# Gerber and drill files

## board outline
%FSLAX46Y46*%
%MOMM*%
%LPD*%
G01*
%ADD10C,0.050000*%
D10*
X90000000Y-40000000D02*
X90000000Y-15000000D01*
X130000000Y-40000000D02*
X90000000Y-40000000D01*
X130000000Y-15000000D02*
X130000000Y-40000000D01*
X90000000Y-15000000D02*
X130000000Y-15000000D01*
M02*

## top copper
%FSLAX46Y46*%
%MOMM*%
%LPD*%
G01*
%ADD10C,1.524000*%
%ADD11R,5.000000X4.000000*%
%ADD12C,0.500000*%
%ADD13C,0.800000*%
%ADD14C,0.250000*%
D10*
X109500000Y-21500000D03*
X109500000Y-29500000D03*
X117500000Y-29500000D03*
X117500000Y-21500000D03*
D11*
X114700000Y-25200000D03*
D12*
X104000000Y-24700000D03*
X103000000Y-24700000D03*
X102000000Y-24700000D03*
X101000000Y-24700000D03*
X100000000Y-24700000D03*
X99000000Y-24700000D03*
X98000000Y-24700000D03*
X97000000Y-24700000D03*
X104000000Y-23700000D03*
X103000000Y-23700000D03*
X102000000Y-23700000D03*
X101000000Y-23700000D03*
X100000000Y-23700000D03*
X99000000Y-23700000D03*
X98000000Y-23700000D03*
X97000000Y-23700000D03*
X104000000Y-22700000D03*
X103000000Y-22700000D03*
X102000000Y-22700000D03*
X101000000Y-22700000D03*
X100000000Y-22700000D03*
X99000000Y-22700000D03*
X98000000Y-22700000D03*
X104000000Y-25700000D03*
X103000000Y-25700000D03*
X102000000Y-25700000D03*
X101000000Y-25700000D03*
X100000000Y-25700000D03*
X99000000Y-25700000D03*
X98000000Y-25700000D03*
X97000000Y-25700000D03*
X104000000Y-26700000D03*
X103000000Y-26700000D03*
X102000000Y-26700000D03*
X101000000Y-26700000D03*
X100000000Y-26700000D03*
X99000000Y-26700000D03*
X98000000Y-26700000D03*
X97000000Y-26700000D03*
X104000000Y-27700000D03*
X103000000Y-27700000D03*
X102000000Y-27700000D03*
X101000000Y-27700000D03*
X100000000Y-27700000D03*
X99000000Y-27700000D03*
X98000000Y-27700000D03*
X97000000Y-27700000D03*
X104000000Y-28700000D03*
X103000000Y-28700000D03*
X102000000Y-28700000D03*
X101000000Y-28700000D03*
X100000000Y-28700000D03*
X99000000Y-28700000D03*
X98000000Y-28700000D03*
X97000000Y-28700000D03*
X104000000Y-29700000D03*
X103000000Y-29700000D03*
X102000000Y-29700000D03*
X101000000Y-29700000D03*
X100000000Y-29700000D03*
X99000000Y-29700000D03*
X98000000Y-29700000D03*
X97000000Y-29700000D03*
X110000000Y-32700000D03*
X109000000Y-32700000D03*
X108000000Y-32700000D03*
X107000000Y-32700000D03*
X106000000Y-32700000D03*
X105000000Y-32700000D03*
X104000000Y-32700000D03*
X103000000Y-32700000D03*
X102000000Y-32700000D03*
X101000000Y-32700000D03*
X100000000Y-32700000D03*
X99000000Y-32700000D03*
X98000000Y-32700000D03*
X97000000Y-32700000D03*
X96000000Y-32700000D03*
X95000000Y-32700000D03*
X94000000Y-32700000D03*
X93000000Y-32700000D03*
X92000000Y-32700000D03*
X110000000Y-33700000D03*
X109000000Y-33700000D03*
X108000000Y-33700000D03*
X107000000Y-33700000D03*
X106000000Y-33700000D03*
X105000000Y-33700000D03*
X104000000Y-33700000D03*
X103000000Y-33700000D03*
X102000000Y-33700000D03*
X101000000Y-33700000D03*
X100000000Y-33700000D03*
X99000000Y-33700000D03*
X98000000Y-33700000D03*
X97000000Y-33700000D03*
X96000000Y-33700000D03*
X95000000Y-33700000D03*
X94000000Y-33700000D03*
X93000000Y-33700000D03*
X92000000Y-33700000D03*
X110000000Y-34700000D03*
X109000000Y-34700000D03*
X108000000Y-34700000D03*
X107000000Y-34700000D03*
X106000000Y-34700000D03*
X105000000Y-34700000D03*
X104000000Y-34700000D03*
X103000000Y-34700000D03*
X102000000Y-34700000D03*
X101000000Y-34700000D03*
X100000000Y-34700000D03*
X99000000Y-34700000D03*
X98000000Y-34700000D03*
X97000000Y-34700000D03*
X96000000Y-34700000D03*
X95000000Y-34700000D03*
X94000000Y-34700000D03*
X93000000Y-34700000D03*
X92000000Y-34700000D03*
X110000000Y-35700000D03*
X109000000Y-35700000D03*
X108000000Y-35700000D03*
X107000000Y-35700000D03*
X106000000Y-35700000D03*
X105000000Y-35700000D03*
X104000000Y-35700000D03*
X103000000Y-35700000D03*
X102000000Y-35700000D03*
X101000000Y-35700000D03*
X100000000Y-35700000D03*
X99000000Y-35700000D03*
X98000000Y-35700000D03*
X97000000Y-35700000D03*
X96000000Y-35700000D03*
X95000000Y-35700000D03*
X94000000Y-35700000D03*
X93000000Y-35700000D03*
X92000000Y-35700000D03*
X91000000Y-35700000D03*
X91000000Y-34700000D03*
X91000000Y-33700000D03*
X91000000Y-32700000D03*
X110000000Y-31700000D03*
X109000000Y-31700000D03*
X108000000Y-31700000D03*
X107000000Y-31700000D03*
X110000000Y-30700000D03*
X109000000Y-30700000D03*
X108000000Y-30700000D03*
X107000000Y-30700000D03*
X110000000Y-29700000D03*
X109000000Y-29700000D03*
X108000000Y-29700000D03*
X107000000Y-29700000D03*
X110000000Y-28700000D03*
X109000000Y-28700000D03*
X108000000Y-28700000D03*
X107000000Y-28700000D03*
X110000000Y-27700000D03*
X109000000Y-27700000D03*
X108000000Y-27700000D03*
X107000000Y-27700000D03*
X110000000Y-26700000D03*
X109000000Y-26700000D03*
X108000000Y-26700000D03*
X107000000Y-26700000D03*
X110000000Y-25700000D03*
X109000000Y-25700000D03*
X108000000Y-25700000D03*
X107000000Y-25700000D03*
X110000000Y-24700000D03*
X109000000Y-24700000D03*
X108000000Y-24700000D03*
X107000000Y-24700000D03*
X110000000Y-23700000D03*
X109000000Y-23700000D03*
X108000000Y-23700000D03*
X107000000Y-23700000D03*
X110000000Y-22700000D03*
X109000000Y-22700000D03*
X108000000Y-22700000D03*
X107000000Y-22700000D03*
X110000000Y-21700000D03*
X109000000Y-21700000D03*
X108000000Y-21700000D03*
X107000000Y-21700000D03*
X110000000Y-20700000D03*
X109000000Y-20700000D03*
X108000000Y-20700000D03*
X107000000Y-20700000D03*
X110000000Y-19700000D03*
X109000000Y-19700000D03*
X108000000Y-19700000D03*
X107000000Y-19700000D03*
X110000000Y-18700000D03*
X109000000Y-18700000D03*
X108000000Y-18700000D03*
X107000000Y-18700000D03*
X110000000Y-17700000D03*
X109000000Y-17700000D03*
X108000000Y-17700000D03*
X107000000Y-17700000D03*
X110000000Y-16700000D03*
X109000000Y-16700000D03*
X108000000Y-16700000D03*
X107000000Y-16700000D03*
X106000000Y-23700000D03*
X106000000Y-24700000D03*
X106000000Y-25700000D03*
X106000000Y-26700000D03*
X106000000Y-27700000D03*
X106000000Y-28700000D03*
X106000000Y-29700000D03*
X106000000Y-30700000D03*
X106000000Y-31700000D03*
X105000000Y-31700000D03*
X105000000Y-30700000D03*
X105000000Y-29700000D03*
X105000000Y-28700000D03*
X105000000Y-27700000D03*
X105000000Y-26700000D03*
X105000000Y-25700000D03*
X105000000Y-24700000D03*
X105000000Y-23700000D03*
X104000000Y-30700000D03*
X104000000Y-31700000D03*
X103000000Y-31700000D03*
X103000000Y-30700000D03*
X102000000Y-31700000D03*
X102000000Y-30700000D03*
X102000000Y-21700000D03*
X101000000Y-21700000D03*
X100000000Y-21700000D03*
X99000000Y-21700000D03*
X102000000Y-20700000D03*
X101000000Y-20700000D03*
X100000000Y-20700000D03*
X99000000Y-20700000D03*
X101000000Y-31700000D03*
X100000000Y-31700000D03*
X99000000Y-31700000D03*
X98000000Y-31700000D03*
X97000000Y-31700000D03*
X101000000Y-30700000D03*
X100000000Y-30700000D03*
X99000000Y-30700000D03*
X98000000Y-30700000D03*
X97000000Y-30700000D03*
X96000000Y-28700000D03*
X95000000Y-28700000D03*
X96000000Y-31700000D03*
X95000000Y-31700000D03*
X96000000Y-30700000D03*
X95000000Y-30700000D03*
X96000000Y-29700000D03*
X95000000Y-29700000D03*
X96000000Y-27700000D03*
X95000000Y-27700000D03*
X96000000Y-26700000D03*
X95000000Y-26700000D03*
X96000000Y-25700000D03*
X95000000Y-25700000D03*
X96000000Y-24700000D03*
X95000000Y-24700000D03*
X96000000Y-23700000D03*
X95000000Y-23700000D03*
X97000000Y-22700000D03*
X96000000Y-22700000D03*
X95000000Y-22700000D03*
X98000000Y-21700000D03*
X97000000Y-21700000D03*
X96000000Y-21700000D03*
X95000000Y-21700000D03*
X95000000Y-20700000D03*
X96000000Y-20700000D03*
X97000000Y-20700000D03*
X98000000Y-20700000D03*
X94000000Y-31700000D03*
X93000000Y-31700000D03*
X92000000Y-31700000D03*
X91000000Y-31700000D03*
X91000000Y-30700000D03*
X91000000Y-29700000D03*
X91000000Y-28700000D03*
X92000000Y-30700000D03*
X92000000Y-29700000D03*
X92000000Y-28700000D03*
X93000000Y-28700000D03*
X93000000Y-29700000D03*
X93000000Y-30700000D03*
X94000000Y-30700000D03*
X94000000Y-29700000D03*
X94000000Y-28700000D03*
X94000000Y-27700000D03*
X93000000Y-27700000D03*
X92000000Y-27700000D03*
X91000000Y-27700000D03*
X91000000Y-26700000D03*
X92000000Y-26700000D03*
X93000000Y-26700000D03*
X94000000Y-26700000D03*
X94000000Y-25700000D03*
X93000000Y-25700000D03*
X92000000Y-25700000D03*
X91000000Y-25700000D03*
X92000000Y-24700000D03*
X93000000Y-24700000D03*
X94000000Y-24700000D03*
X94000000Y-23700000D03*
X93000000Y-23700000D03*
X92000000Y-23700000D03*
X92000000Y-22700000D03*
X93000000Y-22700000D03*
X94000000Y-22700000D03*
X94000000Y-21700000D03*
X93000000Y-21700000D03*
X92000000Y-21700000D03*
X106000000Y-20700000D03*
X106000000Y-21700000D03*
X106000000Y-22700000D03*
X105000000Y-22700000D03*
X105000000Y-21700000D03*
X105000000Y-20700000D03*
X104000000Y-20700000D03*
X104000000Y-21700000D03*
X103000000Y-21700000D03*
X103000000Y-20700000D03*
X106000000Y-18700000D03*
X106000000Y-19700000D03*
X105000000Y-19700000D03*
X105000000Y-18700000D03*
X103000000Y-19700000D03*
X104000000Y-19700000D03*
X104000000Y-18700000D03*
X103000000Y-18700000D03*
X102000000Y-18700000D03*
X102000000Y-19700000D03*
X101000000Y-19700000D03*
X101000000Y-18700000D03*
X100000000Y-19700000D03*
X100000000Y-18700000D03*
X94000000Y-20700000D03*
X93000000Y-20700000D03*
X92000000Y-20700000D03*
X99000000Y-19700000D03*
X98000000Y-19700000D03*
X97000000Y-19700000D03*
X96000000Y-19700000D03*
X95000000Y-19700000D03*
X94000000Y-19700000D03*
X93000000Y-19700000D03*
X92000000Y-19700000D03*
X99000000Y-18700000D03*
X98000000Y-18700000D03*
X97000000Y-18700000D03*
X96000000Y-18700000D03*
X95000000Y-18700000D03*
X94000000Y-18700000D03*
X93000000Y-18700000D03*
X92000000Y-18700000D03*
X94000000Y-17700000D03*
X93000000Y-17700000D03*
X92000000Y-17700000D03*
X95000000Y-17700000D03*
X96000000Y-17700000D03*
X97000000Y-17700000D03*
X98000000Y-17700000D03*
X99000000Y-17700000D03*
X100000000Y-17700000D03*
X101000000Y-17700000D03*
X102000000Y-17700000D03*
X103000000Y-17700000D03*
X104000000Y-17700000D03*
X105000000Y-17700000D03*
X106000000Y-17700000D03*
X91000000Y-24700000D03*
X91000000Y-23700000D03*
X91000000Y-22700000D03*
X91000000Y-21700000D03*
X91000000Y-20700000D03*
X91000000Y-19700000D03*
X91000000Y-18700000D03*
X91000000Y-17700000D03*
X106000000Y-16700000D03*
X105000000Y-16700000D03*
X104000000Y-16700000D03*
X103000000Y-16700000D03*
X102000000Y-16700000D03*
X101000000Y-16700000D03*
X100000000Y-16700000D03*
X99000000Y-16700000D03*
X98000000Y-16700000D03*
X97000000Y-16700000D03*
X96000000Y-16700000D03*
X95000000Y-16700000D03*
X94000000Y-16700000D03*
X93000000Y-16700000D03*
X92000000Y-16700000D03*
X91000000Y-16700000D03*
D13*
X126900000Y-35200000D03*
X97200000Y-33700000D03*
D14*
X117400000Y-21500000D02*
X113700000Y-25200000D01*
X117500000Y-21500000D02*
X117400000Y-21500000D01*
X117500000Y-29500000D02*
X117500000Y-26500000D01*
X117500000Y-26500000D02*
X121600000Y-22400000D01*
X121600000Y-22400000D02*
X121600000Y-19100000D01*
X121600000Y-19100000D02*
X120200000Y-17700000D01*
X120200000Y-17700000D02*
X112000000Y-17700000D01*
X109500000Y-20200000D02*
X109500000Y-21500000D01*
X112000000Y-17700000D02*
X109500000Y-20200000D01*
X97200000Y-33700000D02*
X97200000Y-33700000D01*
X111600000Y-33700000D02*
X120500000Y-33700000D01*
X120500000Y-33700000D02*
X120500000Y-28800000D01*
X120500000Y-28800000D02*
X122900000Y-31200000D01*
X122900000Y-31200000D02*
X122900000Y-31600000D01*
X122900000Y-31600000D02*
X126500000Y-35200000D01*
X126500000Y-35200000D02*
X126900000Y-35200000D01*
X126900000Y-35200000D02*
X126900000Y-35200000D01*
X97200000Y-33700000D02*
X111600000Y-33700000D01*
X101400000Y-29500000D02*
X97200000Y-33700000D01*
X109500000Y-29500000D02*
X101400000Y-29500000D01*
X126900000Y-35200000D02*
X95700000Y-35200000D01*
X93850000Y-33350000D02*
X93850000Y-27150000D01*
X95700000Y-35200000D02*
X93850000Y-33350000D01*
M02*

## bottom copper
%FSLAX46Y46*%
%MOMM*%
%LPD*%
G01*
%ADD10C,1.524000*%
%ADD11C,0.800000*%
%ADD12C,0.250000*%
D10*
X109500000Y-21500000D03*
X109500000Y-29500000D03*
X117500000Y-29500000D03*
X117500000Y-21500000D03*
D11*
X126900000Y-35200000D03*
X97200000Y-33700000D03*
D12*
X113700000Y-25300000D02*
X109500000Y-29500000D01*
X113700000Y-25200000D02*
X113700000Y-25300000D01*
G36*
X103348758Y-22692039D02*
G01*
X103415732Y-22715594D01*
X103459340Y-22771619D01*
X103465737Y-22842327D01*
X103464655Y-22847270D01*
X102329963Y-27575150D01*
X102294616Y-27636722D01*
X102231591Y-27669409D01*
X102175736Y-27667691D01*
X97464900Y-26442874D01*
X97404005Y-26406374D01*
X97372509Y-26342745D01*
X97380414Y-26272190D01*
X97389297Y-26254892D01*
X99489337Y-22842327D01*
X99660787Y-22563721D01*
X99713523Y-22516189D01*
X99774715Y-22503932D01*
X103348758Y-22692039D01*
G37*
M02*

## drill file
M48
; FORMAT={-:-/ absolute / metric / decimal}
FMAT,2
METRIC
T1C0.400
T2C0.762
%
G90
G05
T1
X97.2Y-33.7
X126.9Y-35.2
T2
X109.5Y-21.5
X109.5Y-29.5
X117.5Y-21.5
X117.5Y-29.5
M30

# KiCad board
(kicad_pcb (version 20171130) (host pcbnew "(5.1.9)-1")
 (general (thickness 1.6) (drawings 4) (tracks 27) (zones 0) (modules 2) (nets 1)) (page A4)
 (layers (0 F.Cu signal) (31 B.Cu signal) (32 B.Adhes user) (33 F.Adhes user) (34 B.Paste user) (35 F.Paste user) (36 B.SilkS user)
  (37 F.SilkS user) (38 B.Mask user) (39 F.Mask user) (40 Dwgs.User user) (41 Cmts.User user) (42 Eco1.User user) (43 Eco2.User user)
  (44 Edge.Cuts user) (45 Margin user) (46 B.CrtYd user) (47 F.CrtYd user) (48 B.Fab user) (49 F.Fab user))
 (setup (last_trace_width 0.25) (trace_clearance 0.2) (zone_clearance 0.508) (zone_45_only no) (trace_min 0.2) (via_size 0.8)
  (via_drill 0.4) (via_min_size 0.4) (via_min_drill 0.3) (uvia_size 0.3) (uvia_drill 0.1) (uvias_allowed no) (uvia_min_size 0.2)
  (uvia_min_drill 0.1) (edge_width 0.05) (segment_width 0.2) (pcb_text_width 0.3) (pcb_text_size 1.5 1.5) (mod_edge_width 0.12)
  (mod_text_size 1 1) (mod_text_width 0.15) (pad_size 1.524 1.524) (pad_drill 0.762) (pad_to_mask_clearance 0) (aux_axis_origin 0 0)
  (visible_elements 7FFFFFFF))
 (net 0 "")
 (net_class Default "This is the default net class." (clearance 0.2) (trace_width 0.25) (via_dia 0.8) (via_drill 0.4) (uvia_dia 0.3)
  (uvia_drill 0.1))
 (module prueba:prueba (layer F.Cu) (at 113.5 25.5)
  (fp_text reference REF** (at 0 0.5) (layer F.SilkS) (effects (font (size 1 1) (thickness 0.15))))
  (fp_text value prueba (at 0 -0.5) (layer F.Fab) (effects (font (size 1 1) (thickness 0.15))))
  (pad 5 thru_hole circle (at -4 -4 45) (size 1.524 1.524) (drill 0.762) (layers *.Cu *.Mask))
  (pad 4 thru_hole circle (at -4 4) (size 1.524 1.524) (drill 0.762) (layers *.Cu *.Mask))
  (pad 3 thru_hole circle (at 4 4) (size 1.524 1.524) (drill 0.762) (layers *.Cu *.Mask))
  (pad 2 thru_hole circle (at 4 -4) (size 1.524 1.524) (drill 0.762) (layers *.Cu *.Mask))
  (pad 1 smd rect (at 0.2 -0.3) (size 5 4) (drill (offset 1 0)) (layers F.Cu F.Paste F.Mask) (die_length 1)))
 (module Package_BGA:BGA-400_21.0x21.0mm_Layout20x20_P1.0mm (layer F.Cu) (at 100.5 26.2)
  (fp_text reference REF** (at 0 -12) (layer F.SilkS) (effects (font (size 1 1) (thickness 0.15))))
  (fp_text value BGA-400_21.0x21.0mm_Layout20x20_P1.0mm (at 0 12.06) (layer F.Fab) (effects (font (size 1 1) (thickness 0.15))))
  (pad J14 smd circle (at 3.5 -1.5) (size 0.5 0.5) (layers F.Cu F.Paste F.Mask))
  (pad J13 smd circle (at 2.5 -1.5) (size 0.5 0.5) (layers F.Cu F.Paste F.Mask))
  (pad J12 smd circle (at 1.5 -1.5) (size 0.5 0.5) (layers F.Cu F.Paste F.Mask))
  (pad J11 smd circle (at 0.5 -1.5) (size 0.5 0.5) (layers F.Cu F.Paste F.Mask))
  (pad J10 smd circle (at -0.5 -1.5) (size 0.5 0.5) (layers F.Cu F.Paste F.Mask))
  (pad J9 smd circle (at -1.5 -1.5) (size 0.5 0.5) (layers F.Cu F.Paste F.Mask))
  (pad J8 smd circle (at -2.5 -1.5) (size 0.5 0.5) (layers F.Cu F.Paste F.Mask))
  (pad J7 smd circle (at -3.5 -1.5) (size 0.5 0.5) (layers F.Cu F.Paste F.Mask))
  (pad H14 smd circle (at 3.5 -2.5) (size 0.5 0.5) (layers F.Cu F.Paste F.Mask))
  (pad H13 smd circle (at 2.5 -2.5) (size 0.5 0.5) (layers F.Cu F.Paste F.Mask))
  (pad H12 smd circle (at 1.5 -2.5) (size 0.5 0.5) (layers F.Cu F.Paste F.Mask))
  (pad H11 smd circle (at 0.5 -2.5) (size 0.5 0.5) (layers F.Cu F.Paste F.Mask))
  (pad H10 smd circle (at -0.5 -2.5) (size 0.5 0.5) (layers F.Cu F.Paste F.Mask))
  (pad H9 smd circle (at -1.5 -2.5) (size 0.5 0.5) (layers F.Cu F.Paste F.Mask))
  (pad H8 smd circle (at -2.5 -2.5) (size 0.5 0.5) (layers F.Cu F.Paste F.Mask))
  (pad H7 smd circle (at -3.5 -2.5) (size 0.5 0.5) (layers F.Cu F.Paste F.Mask))
  (pad G14 smd circle (at 3.5 -3.5) (size 0.5 0.5) (layers F.Cu F.Paste F.Mask))
  (pad G13 smd circle (at 2.5 -3.5) (size 0.5 0.5) (layers F.Cu F.Paste F.Mask))
  (pad G12 smd circle (at 1.5 -3.5) (size 0.5 0.5) (layers F.Cu F.Paste F.Mask))
  (pad G11 smd circle (at 0.5 -3.5) (size 0.5 0.5) (layers F.Cu F.Paste F.Mask))
  (pad G10 smd circle (at -0.5 -3.5) (size 0.5 0.5) (layers F.Cu F.Paste F.Mask))
  (pad G9 smd circle (at -1.5 -3.5) (size 0.5 0.5) (layers F.Cu F.Paste F.Mask))
  (pad G8 smd circle (at -2.5 -3.5) (size 0.5 0.5) (layers F.Cu F.Paste F.Mask))
  (pad K14 smd circle (at 3.5 -0.5) (size 0.5 0.5) (layers F.Cu F.Paste F.Mask))
  (pad K13 smd circle (at 2.5 -0.5) (size 0.5 0.5) (layers F.Cu F.Paste F.Mask))
  (pad K12 smd circle (at 1.5 -0.5) (size 0.5 0.5) (layers F.Cu F.Paste F.Mask))
  (pad K11 smd circle (at 0.5 -0.5) (size 0.5 0.5) (layers F.Cu F.Paste F.Mask))
  (pad K10 smd circle (at -0.5 -0.5) (size 0.5 0.5) (layers F.Cu F.Paste F.Mask))
  (pad K9 smd circle (at -1.5 -0.5) (size 0.5 0.5) (layers F.Cu F.Paste F.Mask))
  (pad K8 smd circle (at -2.5 -0.5) (size 0.5 0.5) (layers F.Cu F.Paste F.Mask))
  (pad K7 smd circle (at -3.5 -0.5) (size 0.5 0.5) (layers F.Cu F.Paste F.Mask))
  (pad L14 smd circle (at 3.5 0.5) (size 0.5 0.5) (layers F.Cu F.Paste F.Mask))
  (pad L13 smd circle (at 2.5 0.5) (size 0.5 0.5) (layers F.Cu F.Paste F.Mask))
  (pad L12 smd circle (at 1.5 0.5) (size 0.5 0.5) (layers F.Cu F.Paste F.Mask))
  (pad L11 smd circle (at 0.5 0.5) (size 0.5 0.5) (layers F.Cu F.Paste F.Mask))
  (pad L10 smd circle (at -0.5 0.5) (size 0.5 0.5) (layers F.Cu F.Paste F.Mask))
  (pad L9 smd circle (at -1.5 0.5) (size 0.5 0.5) (layers F.Cu F.Paste F.Mask))
  (pad L8 smd circle (at -2.5 0.5) (size 0.5 0.5) (layers F.Cu F.Paste F.Mask))
  (pad L7 smd circle (at -3.5 0.5) (size 0.5 0.5) (layers F.Cu F.Paste F.Mask))
  (pad M14 smd circle (at 3.5 1.5) (size 0.5 0.5) (layers F.Cu F.Paste F.Mask))
  (pad M13 smd circle (at 2.5 1.5) (size 0.5 0.5) (layers F.Cu F.Paste F.Mask))
  (pad M12 smd circle (at 1.5 1.5) (size 0.5 0.5) (layers F.Cu F.Paste F.Mask))
  (pad M11 smd circle (at 0.5 1.5) (size 0.5 0.5) (layers F.Cu F.Paste F.Mask))
  (pad M10 smd circle (at -0.5 1.5) (size 0.5 0.5) (layers F.Cu F.Paste F.Mask))
  (pad M9 smd circle (at -1.5 1.5) (size 0.5 0.5) (layers F.Cu F.Paste F.Mask))
  (pad M8 smd circle (at -2.5 1.5) (size 0.5 0.5) (layers F.Cu F.Paste F.Mask))
  (pad M7 smd circle (at -3.5 1.5) (size 0.5 0.5) (layers F.Cu F.Paste F.Mask))
  (pad N14 smd circle (at 3.5 2.5) (size 0.5 0.5) (layers F.Cu F.Paste F.Mask))
  (pad N13 smd circle (at 2.5 2.5) (size 0.5 0.5) (layers F.Cu F.Paste F.Mask))
  (pad N12 smd circle (at 1.5 2.5) (size 0.5 0.5) (layers F.Cu F.Paste F.Mask))
  (pad N11 smd circle (at 0.5 2.5) (size 0.5 0.5) (layers F.Cu F.Paste F.Mask))
  (pad N10 smd circle (at -0.5 2.5) (size 0.5 0.5) (layers F.Cu F.Paste F.Mask))
  (pad N9 smd circle (at -1.5 2.5) (size 0.5 0.5) (layers F.Cu F.Paste F.Mask))
  (pad N8 smd circle (at -2.5 2.5) (size 0.5 0.5) (layers F.Cu F.Paste F.Mask))
  (pad N7 smd circle (at -3.5 2.5) (size 0.5 0.5) (layers F.Cu F.Paste F.Mask))
  (pad P14 smd circle (at 3.5 3.5) (size 0.5 0.5) (layers F.Cu F.Paste F.Mask))
  (pad P13 smd circle (at 2.5 3.5) (size 0.5 0.5) (layers F.Cu F.Paste F.Mask))
  (pad P12 smd circle (at 1.5 3.5) (size 0.5 0.5) (layers F.Cu F.Paste F.Mask))
  (pad P11 smd circle (at 0.5 3.5) (size 0.5 0.5) (layers F.Cu F.Paste F.Mask))
  (pad P10 smd circle (at -0.5 3.5) (size 0.5 0.5) (layers F.Cu F.Paste F.Mask))
  (pad P9 smd circle (at -1.5 3.5) (size 0.5 0.5) (layers F.Cu F.Paste F.Mask))
  (pad P8 smd circle (at -2.5 3.5) (size 0.5 0.5) (layers F.Cu F.Paste F.Mask))
  (pad P7 smd circle (at -3.5 3.5) (size 0.5 0.5) (layers F.Cu F.Paste F.Mask))
  (pad U20 smd circle (at 9.5 6.5) (size 0.5 0.5) (layers F.Cu F.Paste F.Mask))
  (pad U19 smd circle (at 8.5 6.5) (size 0.5 0.5) (layers F.Cu F.Paste F.Mask))
  (pad U18 smd circle (at 7.5 6.5) (size 0.5 0.5) (layers F.Cu F.Paste F.Mask))
  (pad U17 smd circle (at 6.5 6.5) (size 0.5 0.5) (layers F.Cu F.Paste F.Mask))
  (pad U16 smd circle (at 5.5 6.5) (size 0.5 0.5) (layers F.Cu F.Paste F.Mask))
  (pad U15 smd circle (at 4.5 6.5) (size 0.5 0.5) (layers F.Cu F.Paste F.Mask))
  (pad U14 smd circle (at 3.5 6.5) (size 0.5 0.5) (layers F.Cu F.Paste F.Mask))
  (pad U13 smd circle (at 2.5 6.5) (size 0.5 0.5) (layers F.Cu F.Paste F.Mask))
  (pad U12 smd circle (at 1.5 6.5) (size 0.5 0.5) (layers F.Cu F.Paste F.Mask))
  (pad U11 smd circle (at 0.5 6.5) (size 0.5 0.5) (layers F.Cu F.Paste F.Mask))
  (pad U10 smd circle (at -0.5 6.5) (size 0.5 0.5) (layers F.Cu F.Paste F.Mask))
  (pad U9 smd circle (at -1.5 6.5) (size 0.5 0.5) (layers F.Cu F.Paste F.Mask))
  (pad U8 smd circle (at -2.5 6.5) (size 0.5 0.5) (layers F.Cu F.Paste F.Mask))
  (pad U7 smd circle (at -3.5 6.5) (size 0.5 0.5) (layers F.Cu F.Paste F.Mask))
  (pad U6 smd circle (at -4.5 6.5) (size 0.5 0.5) (layers F.Cu F.Paste F.Mask))
  (pad U5 smd circle (at -5.5 6.5) (size 0.5 0.5) (layers F.Cu F.Paste F.Mask))
  (pad U4 smd circle (at -6.5 6.5) (size 0.5 0.5) (layers F.Cu F.Paste F.Mask))
  (pad U3 smd circle (at -7.5 6.5) (size 0.5 0.5) (layers F.Cu F.Paste F.Mask))
  (pad U2 smd circle (at -8.5 6.5) (size 0.5 0.5) (layers F.Cu F.Paste F.Mask))
  (pad V20 smd circle (at 9.5 7.5) (size 0.5 0.5) (layers F.Cu F.Paste F.Mask))
  (pad V19 smd circle (at 8.5 7.5) (size 0.5 0.5) (layers F.Cu F.Paste F.Mask))
  (pad V18 smd circle (at 7.5 7.5) (size 0.5 0.5) (layers F.Cu F.Paste F.Mask))
  (pad V17 smd circle (at 6.5 7.5) (size 0.5 0.5) (layers F.Cu F.Paste F.Mask))
  (pad V16 smd circle (at 5.5 7.5) (size 0.5 0.5) (layers F.Cu F.Paste F.Mask))
  (pad V15 smd circle (at 4.5 7.5) (size 0.5 0.5) (layers F.Cu F.Paste F.Mask))
  (pad V14 smd circle (at 3.5 7.5) (size 0.5 0.5) (layers F.Cu F.Paste F.Mask))
  (pad V13 smd circle (at 2.5 7.5) (size 0.5 0.5) (layers F.Cu F.Paste F.Mask))
  (pad V12 smd circle (at 1.5 7.5) (size 0.5 0.5) (layers F.Cu F.Paste F.Mask))
  (pad V11 smd circle (at 0.5 7.5) (size 0.5 0.5) (layers F.Cu F.Paste F.Mask))
  (pad V10 smd circle (at -0.5 7.5) (size 0.5 0.5) (layers F.Cu F.Paste F.Mask))
  (pad V9 smd circle (at -1.5 7.5) (size 0.5 0.5) (layers F.Cu F.Paste F.Mask))
  (pad V8 smd circle (at -2.5 7.5) (size 0.5 0.5) (layers F.Cu F.Paste F.Mask))
  (pad V7 smd circle (at -3.5 7.5) (size 0.5 0.5) (layers F.Cu F.Paste F.Mask))
  (pad V6 smd circle (at -4.5 7.5) (size 0.5 0.5) (layers F.Cu F.Paste F.Mask))
  (pad V5 smd circle (at -5.5 7.5) (size 0.5 0.5) (layers F.Cu F.Paste F.Mask))
  (pad V4 smd circle (at -6.5 7.5) (size 0.5 0.5) (layers F.Cu F.Paste F.Mask))
  (pad V3 smd circle (at -7.5 7.5) (size 0.5 0.5) (layers F.Cu F.Paste F.Mask))
  (pad V2 smd circle (at -8.5 7.5) (size 0.5 0.5) (layers F.Cu F.Paste F.Mask))
  (pad W20 smd circle (at 9.5 8.5) (size 0.5 0.5) (layers F.Cu F.Paste F.Mask))
  (pad W19 smd circle (at 8.5 8.5) (size 0.5 0.5) (layers F.Cu F.Paste F.Mask))
  (pad W18 smd circle (at 7.5 8.5) (size 0.5 0.5) (layers F.Cu F.Paste F.Mask))
  (pad W17 smd circle (at 6.5 8.5) (size 0.5 0.5) (layers F.Cu F.Paste F.Mask))
  (pad W16 smd circle (at 5.5 8.5) (size 0.5 0.5) (layers F.Cu F.Paste F.Mask))
  (pad W15 smd circle (at 4.5 8.5) (size 0.5 0.5) (layers F.Cu F.Paste F.Mask))
  (pad W14 smd circle (at 3.5 8.5) (size 0.5 0.5) (layers F.Cu F.Paste F.Mask))
  (pad W13 smd circle (at 2.5 8.5) (size 0.5 0.5) (layers F.Cu F.Paste F.Mask))
  (pad W12 smd circle (at 1.5 8.5) (size 0.5 0.5) (layers F.Cu F.Paste F.Mask))
  (pad W11 smd circle (at 0.5 8.5) (size 0.5 0.5) (layers F.Cu F.Paste F.Mask))
  (pad W10 smd circle (at -0.5 8.5) (size 0.5 0.5) (layers F.Cu F.Paste F.Mask))
  (pad W9 smd circle (at -1.5 8.5) (size 0.5 0.5) (layers F.Cu F.Paste F.Mask))
  (pad W8 smd circle (at -2.5 8.5) (size 0.5 0.5) (layers F.Cu F.Paste F.Mask))
  (pad W7 smd circle (at -3.5 8.5) (size 0.5 0.5) (layers F.Cu F.Paste F.Mask))
  (pad W6 smd circle (at -4.5 8.5) (size 0.5 0.5) (layers F.Cu F.Paste F.Mask))
  (pad W5 smd circle (at -5.5 8.5) (size 0.5 0.5) (layers F.Cu F.Paste F.Mask))
  (pad W4 smd circle (at -6.5 8.5) (size 0.5 0.5) (layers F.Cu F.Paste F.Mask))
  (pad W3 smd circle (at -7.5 8.5) (size 0.5 0.5) (layers F.Cu F.Paste F.Mask))
  (pad W2 smd circle (at -8.5 8.5) (size 0.5 0.5) (layers F.Cu F.Paste F.Mask))
  (pad Y20 smd circle (at 9.5 9.5) (size 0.5 0.5) (layers F.Cu F.Paste F.Mask))
  (pad Y19 smd circle (at 8.5 9.5) (size 0.5 0.5) (layers F.Cu F.Paste F.Mask))
  (pad Y18 smd circle (at 7.5 9.5) (size 0.5 0.5) (layers F.Cu F.Paste F.Mask))
  (pad Y17 smd circle (at 6.5 9.5) (size 0.5 0.5) (layers F.Cu F.Paste F.Mask))
  (pad Y16 smd circle (at 5.5 9.5) (size 0.5 0.5) (layers F.Cu F.Paste F.Mask))
  (pad Y15 smd circle (at 4.5 9.5) (size 0.5 0.5) (layers F.Cu F.Paste F.Mask))
  (pad Y14 smd circle (at 3.5 9.5) (size 0.5 0.5) (layers F.Cu F.Paste F.Mask))
  (pad Y13 smd circle (at 2.5 9.5) (size 0.5 0.5) (layers F.Cu F.Paste F.Mask))
  (pad Y12 smd circle (at 1.5 9.5) (size 0.5 0.5) (layers F.Cu F.Paste F.Mask))
  (pad Y11 smd circle (at 0.5 9.5) (size 0.5 0.5) (layers F.Cu F.Paste F.Mask))
  (pad Y10 smd circle (at -0.5 9.5) (size 0.5 0.5) (layers F.Cu F.Paste F.Mask))
  (pad Y9 smd circle (at -1.5 9.5) (size 0.5 0.5) (layers F.Cu F.Paste F.Mask))
  (pad Y8 smd circle (at -2.5 9.5) (size 0.5 0.5) (layers F.Cu F.Paste F.Mask))
  (pad Y7 smd circle (at -3.5 9.5) (size 0.5 0.5) (layers F.Cu F.Paste F.Mask))
  (pad Y6 smd circle (at -4.5 9.5) (size 0.5 0.5) (layers F.Cu F.Paste F.Mask))
  (pad Y5 smd circle (at -5.5 9.5) (size 0.5 0.5) (layers F.Cu F.Paste F.Mask))
  (pad Y4 smd circle (at -6.5 9.5) (size 0.5 0.5) (layers F.Cu F.Paste F.Mask))
  (pad Y3 smd circle (at -7.5 9.5) (size 0.5 0.5) (layers F.Cu F.Paste F.Mask))
  (pad Y2 smd circle (at -8.5 9.5) (size 0.5 0.5) (layers F.Cu F.Paste F.Mask))
  (pad Y1 smd circle (at -9.5 9.5) (size 0.5 0.5) (layers F.Cu F.Paste F.Mask))
  (pad W1 smd circle (at -9.5 8.5) (size 0.5 0.5) (layers F.Cu F.Paste F.Mask))
  (pad V1 smd circle (at -9.5 7.5) (size 0.5 0.5) (layers F.Cu F.Paste F.Mask))
  (pad U1 smd circle (at -9.5 6.5) (size 0.5 0.5) (layers F.Cu F.Paste F.Mask))
  (pad T20 smd circle (at 9.5 5.5) (size 0.5 0.5) (layers F.Cu F.Paste F.Mask))
  (pad T19 smd circle (at 8.5 5.5) (size 0.5 0.5) (layers F.Cu F.Paste F.Mask))
  (pad T18 smd circle (at 7.5 5.5) (size 0.5 0.5) (layers F.Cu F.Paste F.Mask))
  (pad T17 smd circle (at 6.5 5.5) (size 0.5 0.5) (layers F.Cu F.Paste F.Mask))
  (pad R20 smd circle (at 9.5 4.5) (size 0.5 0.5) (layers F.Cu F.Paste F.Mask))
  (pad R19 smd circle (at 8.5 4.5) (size 0.5 0.5) (layers F.Cu F.Paste F.Mask))
  (pad R18 smd circle (at 7.5 4.5) (size 0.5 0.5) (layers F.Cu F.Paste F.Mask))
  (pad R17 smd circle (at 6.5 4.5) (size 0.5 0.5) (layers F.Cu F.Paste F.Mask))
  (pad P20 smd circle (at 9.5 3.5) (size 0.5 0.5) (layers F.Cu F.Paste F.Mask))
  (pad P19 smd circle (at 8.5 3.5) (size 0.5 0.5) (layers F.Cu F.Paste F.Mask))
  (pad P18 smd circle (at 7.5 3.5) (size 0.5 0.5) (layers F.Cu F.Paste F.Mask))
  (pad P17 smd circle (at 6.5 3.5) (size 0.5 0.5) (layers F.Cu F.Paste F.Mask))
  (pad N20 smd circle (at 9.5 2.5) (size 0.5 0.5) (layers F.Cu F.Paste F.Mask))
  (pad N19 smd circle (at 8.5 2.5) (size 0.5 0.5) (layers F.Cu F.Paste F.Mask))
  (pad N18 smd circle (at 7.5 2.5) (size 0.5 0.5) (layers F.Cu F.Paste F.Mask))
  (pad N17 smd circle (at 6.5 2.5) (size 0.5 0.5) (layers F.Cu F.Paste F.Mask))
  (pad M20 smd circle (at 9.5 1.5) (size 0.5 0.5) (layers F.Cu F.Paste F.Mask))
  (pad M19 smd circle (at 8.5 1.5) (size 0.5 0.5) (layers F.Cu F.Paste F.Mask))
  (pad M18 smd circle (at 7.5 1.5) (size 0.5 0.5) (layers F.Cu F.Paste F.Mask))
  (pad M17 smd circle (at 6.5 1.5) (size 0.5 0.5) (layers F.Cu F.Paste F.Mask))
  (pad L20 smd circle (at 9.5 0.5) (size 0.5 0.5) (layers F.Cu F.Paste F.Mask))
  (pad L19 smd circle (at 8.5 0.5) (size 0.5 0.5) (layers F.Cu F.Paste F.Mask))
  (pad L18 smd circle (at 7.5 0.5) (size 0.5 0.5) (layers F.Cu F.Paste F.Mask))
  (pad L17 smd circle (at 6.5 0.5) (size 0.5 0.5) (layers F.Cu F.Paste F.Mask))
  (pad K20 smd circle (at 9.5 -0.5) (size 0.5 0.5) (layers F.Cu F.Paste F.Mask))
  (pad K19 smd circle (at 8.5 -0.5) (size 0.5 0.5) (layers F.Cu F.Paste F.Mask))
  (pad K18 smd circle (at 7.5 -0.5) (size 0.5 0.5) (layers F.Cu F.Paste F.Mask))
  (pad K17 smd circle (at 6.5 -0.5) (size 0.5 0.5) (layers F.Cu F.Paste F.Mask))
  (pad J20 smd circle (at 9.5 -1.5) (size 0.5 0.5) (layers F.Cu F.Paste F.Mask))
  (pad J19 smd circle (at 8.5 -1.5) (size 0.5 0.5) (layers F.Cu F.Paste F.Mask))
  (pad J18 smd circle (at 7.5 -1.5) (size 0.5 0.5) (layers F.Cu F.Paste F.Mask))
  (pad J17 smd circle (at 6.5 -1.5) (size 0.5 0.5) (layers F.Cu F.Paste F.Mask))
  (pad H20 smd circle (at 9.5 -2.5) (size 0.5 0.5) (layers F.Cu F.Paste F.Mask))
  (pad H19 smd circle (at 8.5 -2.5) (size 0.5 0.5) (layers F.Cu F.Paste F.Mask))
  (pad H18 smd circle (at 7.5 -2.5) (size 0.5 0.5) (layers F.Cu F.Paste F.Mask))
  (pad H17 smd circle (at 6.5 -2.5) (size 0.5 0.5) (layers F.Cu F.Paste F.Mask))
  (pad G20 smd circle (at 9.5 -3.5) (size 0.5 0.5) (layers F.Cu F.Paste F.Mask))
  (pad G19 smd circle (at 8.5 -3.5) (size 0.5 0.5) (layers F.Cu F.Paste F.Mask))
  (pad G18 smd circle (at 7.5 -3.5) (size 0.5 0.5) (layers F.Cu F.Paste F.Mask))
  (pad G17 smd circle (at 6.5 -3.5) (size 0.5 0.5) (layers F.Cu F.Paste F.Mask))
  (pad F20 smd circle (at 9.5 -4.5) (size 0.5 0.5) (layers F.Cu F.Paste F.Mask))
  (pad F19 smd circle (at 8.5 -4.5) (size 0.5 0.5) (layers F.Cu F.Paste F.Mask))
  (pad F18 smd circle (at 7.5 -4.5) (size 0.5 0.5) (layers F.Cu F.Paste F.Mask))
  (pad F17 smd circle (at 6.5 -4.5) (size 0.5 0.5) (layers F.Cu F.Paste F.Mask))
  (pad E20 smd circle (at 9.5 -5.5) (size 0.5 0.5) (layers F.Cu F.Paste F.Mask))
  (pad E19 smd circle (at 8.5 -5.5) (size 0.5 0.5) (layers F.Cu F.Paste F.Mask))
  (pad E18 smd circle (at 7.5 -5.5) (size 0.5 0.5) (layers F.Cu F.Paste F.Mask))
  (pad E17 smd circle (at 6.5 -5.5) (size 0.5 0.5) (layers F.Cu F.Paste F.Mask))
  (pad D20 smd circle (at 9.5 -6.5) (size 0.5 0.5) (layers F.Cu F.Paste F.Mask))
  (pad D19 smd circle (at 8.5 -6.5) (size 0.5 0.5) (layers F.Cu F.Paste F.Mask))
  (pad D18 smd circle (at 7.5 -6.5) (size 0.5 0.5) (layers F.Cu F.Paste F.Mask))
  (pad D17 smd circle (at 6.5 -6.5) (size 0.5 0.5) (layers F.Cu F.Paste F.Mask))
  (pad C20 smd circle (at 9.5 -7.5) (size 0.5 0.5) (layers F.Cu F.Paste F.Mask))
  (pad C19 smd circle (at 8.5 -7.5) (size 0.5 0.5) (layers F.Cu F.Paste F.Mask))
  (pad C18 smd circle (at 7.5 -7.5) (size 0.5 0.5) (layers F.Cu F.Paste F.Mask))
  (pad C17 smd circle (at 6.5 -7.5) (size 0.5 0.5) (layers F.Cu F.Paste F.Mask))
  (pad B20 smd circle (at 9.5 -8.5) (size 0.5 0.5) (layers F.Cu F.Paste F.Mask))
  (pad B19 smd circle (at 8.5 -8.5) (size 0.5 0.5) (layers F.Cu F.Paste F.Mask))
  (pad B18 smd circle (at 7.5 -8.5) (size 0.5 0.5) (layers F.Cu F.Paste F.Mask))
  (pad B17 smd circle (at 6.5 -8.5) (size 0.5 0.5) (layers F.Cu F.Paste F.Mask))
  (pad A20 smd circle (at 9.5 -9.5) (size 0.5 0.5) (layers F.Cu F.Paste F.Mask))
  (pad A19 smd circle (at 8.5 -9.5) (size 0.5 0.5) (layers F.Cu F.Paste F.Mask))
  (pad A18 smd circle (at 7.5 -9.5) (size 0.5 0.5) (layers F.Cu F.Paste F.Mask))
  (pad A17 smd circle (at 6.5 -9.5) (size 0.5 0.5) (layers F.Cu F.Paste F.Mask))
  (pad H16 smd circle (at 5.5 -2.5) (size 0.5 0.5) (layers F.Cu F.Paste F.Mask))
  (pad J16 smd circle (at 5.5 -1.5) (size 0.5 0.5) (layers F.Cu F.Paste F.Mask))
  (pad K16 smd circle (at 5.5 -0.5) (size 0.5 0.5) (layers F.Cu F.Paste F.Mask))
  (pad L16 smd circle (at 5.5 0.5) (size 0.5 0.5) (layers F.Cu F.Paste F.Mask))
  (pad M16 smd circle (at 5.5 1.5) (size 0.5 0.5) (layers F.Cu F.Paste F.Mask))
  (pad N16 smd circle (at 5.5 2.5) (size 0.5 0.5) (layers F.Cu F.Paste F.Mask))
  (pad P16 smd circle (at 5.5 3.5) (size 0.5 0.5) (layers F.Cu F.Paste F.Mask))
  (pad R16 smd circle (at 5.5 4.5) (size 0.5 0.5) (layers F.Cu F.Paste F.Mask))
  (pad T16 smd circle (at 5.5 5.5) (size 0.5 0.5) (layers F.Cu F.Paste F.Mask))
  (pad T15 smd circle (at 4.5 5.5) (size 0.5 0.5) (layers F.Cu F.Paste F.Mask))
  (pad R15 smd circle (at 4.5 4.5) (size 0.5 0.5) (layers F.Cu F.Paste F.Mask))
  (pad P15 smd circle (at 4.5 3.5) (size 0.5 0.5) (layers F.Cu F.Paste F.Mask))
  (pad N15 smd circle (at 4.5 2.5) (size 0.5 0.5) (layers F.Cu F.Paste F.Mask))
  (pad M15 smd circle (at 4.5 1.5) (size 0.5 0.5) (layers F.Cu F.Paste F.Mask))
  (pad L15 smd circle (at 4.5 0.5) (size 0.5 0.5) (layers F.Cu F.Paste F.Mask))
  (pad K15 smd circle (at 4.5 -0.5) (size 0.5 0.5) (layers F.Cu F.Paste F.Mask))
  (pad J15 smd circle (at 4.5 -1.5) (size 0.5 0.5) (layers F.Cu F.Paste F.Mask))
  (pad H15 smd circle (at 4.5 -2.5) (size 0.5 0.5) (layers F.Cu F.Paste F.Mask))
  (pad R14 smd circle (at 3.5 4.5) (size 0.5 0.5) (layers F.Cu F.Paste F.Mask))
  (pad T14 smd circle (at 3.5 5.5) (size 0.5 0.5) (layers F.Cu F.Paste F.Mask))
  (pad T13 smd circle (at 2.5 5.5) (size 0.5 0.5) (layers F.Cu F.Paste F.Mask))
  (pad R13 smd circle (at 2.5 4.5) (size 0.5 0.5) (layers F.Cu F.Paste F.Mask))
  (pad T12 smd circle (at 1.5 5.5) (size 0.5 0.5) (layers F.Cu F.Paste F.Mask))
  (pad R12 smd circle (at 1.5 4.5) (size 0.5 0.5) (layers F.Cu F.Paste F.Mask))
  (pad F12 smd circle (at 1.5 -4.5) (size 0.5 0.5) (layers F.Cu F.Paste F.Mask))
  (pad F11 smd circle (at 0.5 -4.5) (size 0.5 0.5) (layers F.Cu F.Paste F.Mask))
  (pad F10 smd circle (at -0.5 -4.5) (size 0.5 0.5) (layers F.Cu F.Paste F.Mask))
  (pad F9 smd circle (at -1.5 -4.5) (size 0.5 0.5) (layers F.Cu F.Paste F.Mask))
  (pad E12 smd circle (at 1.5 -5.5) (size 0.5 0.5) (layers F.Cu F.Paste F.Mask))
  (pad E11 smd circle (at 0.5 -5.5) (size 0.5 0.5) (layers F.Cu F.Paste F.Mask))
  (pad E10 smd circle (at -0.5 -5.5) (size 0.5 0.5) (layers F.Cu F.Paste F.Mask))
  (pad E9 smd circle (at -1.5 -5.5) (size 0.5 0.5) (layers F.Cu F.Paste F.Mask))
  (pad T11 smd circle (at 0.5 5.5) (size 0.5 0.5) (layers F.Cu F.Paste F.Mask))
  (pad T10 smd circle (at -0.5 5.5) (size 0.5 0.5) (layers F.Cu F.Paste F.Mask))
  (pad T9 smd circle (at -1.5 5.5) (size 0.5 0.5) (layers F.Cu F.Paste F.Mask))
  (pad T8 smd circle (at -2.5 5.5) (size 0.5 0.5) (layers F.Cu F.Paste F.Mask))
  (pad T7 smd circle (at -3.5 5.5) (size 0.5 0.5) (layers F.Cu F.Paste F.Mask))
  (pad R11 smd circle (at 0.5 4.5) (size 0.5 0.5) (layers F.Cu F.Paste F.Mask))
  (pad R10 smd circle (at -0.5 4.5) (size 0.5 0.5) (layers F.Cu F.Paste F.Mask))
  (pad R9 smd circle (at -1.5 4.5) (size 0.5 0.5) (layers F.Cu F.Paste F.Mask))
  (pad R8 smd circle (at -2.5 4.5) (size 0.5 0.5) (layers F.Cu F.Paste F.Mask))
  (pad R7 smd circle (at -3.5 4.5) (size 0.5 0.5) (layers F.Cu F.Paste F.Mask))
  (pad N6 smd circle (at -4.5 2.5) (size 0.5 0.5) (layers F.Cu F.Paste F.Mask))
  (pad N5 smd circle (at -5.5 2.5) (size 0.5 0.5) (layers F.Cu F.Paste F.Mask))
  (pad T6 smd circle (at -4.5 5.5) (size 0.5 0.5) (layers F.Cu F.Paste F.Mask))
  (pad T5 smd circle (at -5.5 5.5) (size 0.5 0.5) (layers F.Cu F.Paste F.Mask))
  (pad R6 smd circle (at -4.5 4.5) (size 0.5 0.5) (layers F.Cu F.Paste F.Mask))
  (pad R5 smd circle (at -5.5 4.5) (size 0.5 0.5) (layers F.Cu F.Paste F.Mask))
  (pad P6 smd circle (at -4.5 3.5) (size 0.5 0.5) (layers F.Cu F.Paste F.Mask))
  (pad P5 smd circle (at -5.5 3.5) (size 0.5 0.5) (layers F.Cu F.Paste F.Mask))
  (pad M6 smd circle (at -4.5 1.5) (size 0.5 0.5) (layers F.Cu F.Paste F.Mask))
  (pad M5 smd circle (at -5.5 1.5) (size 0.5 0.5) (layers F.Cu F.Paste F.Mask))
  (pad L6 smd circle (at -4.5 0.5) (size 0.5 0.5) (layers F.Cu F.Paste F.Mask))
  (pad L5 smd circle (at -5.5 0.5) (size 0.5 0.5) (layers F.Cu F.Paste F.Mask))
  (pad K6 smd circle (at -4.5 -0.5) (size 0.5 0.5) (layers F.Cu F.Paste F.Mask))
  (pad K5 smd circle (at -5.5 -0.5) (size 0.5 0.5) (layers F.Cu F.Paste F.Mask))
  (pad J6 smd circle (at -4.5 -1.5) (size 0.5 0.5) (layers F.Cu F.Paste F.Mask))
  (pad J5 smd circle (at -5.5 -1.5) (size 0.5 0.5) (layers F.Cu F.Paste F.Mask))
  (pad H6 smd circle (at -4.5 -2.5) (size 0.5 0.5) (layers F.Cu F.Paste F.Mask))
  (pad H5 smd circle (at -5.5 -2.5) (size 0.5 0.5) (layers F.Cu F.Paste F.Mask))
  (pad G7 smd circle (at -3.5 -3.5) (size 0.5 0.5) (layers F.Cu F.Paste F.Mask))
  (pad G6 smd circle (at -4.5 -3.5) (size 0.5 0.5) (layers F.Cu F.Paste F.Mask))
  (pad G5 smd circle (at -5.5 -3.5) (size 0.5 0.5) (layers F.Cu F.Paste F.Mask))
  (pad F8 smd circle (at -2.5 -4.5) (size 0.5 0.5) (layers F.Cu F.Paste F.Mask))
  (pad F7 smd circle (at -3.5 -4.5) (size 0.5 0.5) (layers F.Cu F.Paste F.Mask))
  (pad F6 smd circle (at -4.5 -4.5) (size 0.5 0.5) (layers F.Cu F.Paste F.Mask))
  (pad F5 smd circle (at -5.5 -4.5) (size 0.5 0.5) (layers F.Cu F.Paste F.Mask))
  (pad E5 smd circle (at -5.5 -5.5) (size 0.5 0.5) (layers F.Cu F.Paste F.Mask))
  (pad E6 smd circle (at -4.5 -5.5) (size 0.5 0.5) (layers F.Cu F.Paste F.Mask))
  (pad E7 smd circle (at -3.5 -5.5) (size 0.5 0.5) (layers F.Cu F.Paste F.Mask))
  (pad E8 smd circle (at -2.5 -5.5) (size 0.5 0.5) (layers F.Cu F.Paste F.Mask))
  (pad T4 smd circle (at -6.5 5.5) (size 0.5 0.5) (layers F.Cu F.Paste F.Mask))
  (pad T3 smd circle (at -7.5 5.5) (size 0.5 0.5) (layers F.Cu F.Paste F.Mask))
  (pad T2 smd circle (at -8.5 5.5) (size 0.5 0.5) (layers F.Cu F.Paste F.Mask))
  (pad T1 smd circle (at -9.5 5.5) (size 0.5 0.5) (layers F.Cu F.Paste F.Mask))
  (pad R1 smd circle (at -9.5 4.5) (size 0.5 0.5) (layers F.Cu F.Paste F.Mask))
  (pad P1 smd circle (at -9.5 3.5) (size 0.5 0.5) (layers F.Cu F.Paste F.Mask))
  (pad N1 smd circle (at -9.5 2.5) (size 0.5 0.5) (layers F.Cu F.Paste F.Mask))
  (pad R2 smd circle (at -8.5 4.5) (size 0.5 0.5) (layers F.Cu F.Paste F.Mask))
  (pad P2 smd circle (at -8.5 3.5) (size 0.5 0.5) (layers F.Cu F.Paste F.Mask))
  (pad N2 smd circle (at -8.5 2.5) (size 0.5 0.5) (layers F.Cu F.Paste F.Mask))
  (pad N3 smd circle (at -7.5 2.5) (size 0.5 0.5) (layers F.Cu F.Paste F.Mask))
  (pad P3 smd circle (at -7.5 3.5) (size 0.5 0.5) (layers F.Cu F.Paste F.Mask))
  (pad R3 smd circle (at -7.5 4.5) (size 0.5 0.5) (layers F.Cu F.Paste F.Mask))
  (pad R4 smd circle (at -6.5 4.5) (size 0.5 0.5) (layers F.Cu F.Paste F.Mask))
  (pad P4 smd circle (at -6.5 3.5) (size 0.5 0.5) (layers F.Cu F.Paste F.Mask))
  (pad N4 smd circle (at -6.5 2.5) (size 0.5 0.5) (layers F.Cu F.Paste F.Mask))
  (pad M4 smd circle (at -6.5 1.5) (size 0.5 0.5) (layers F.Cu F.Paste F.Mask))
  (pad M3 smd circle (at -7.5 1.5) (size 0.5 0.5) (layers F.Cu F.Paste F.Mask))
  (pad M2 smd circle (at -8.5 1.5) (size 0.5 0.5) (layers F.Cu F.Paste F.Mask))
  (pad M1 smd circle (at -9.5 1.5) (size 0.5 0.5) (layers F.Cu F.Paste F.Mask))
  (pad L1 smd circle (at -9.5 0.5) (size 0.5 0.5) (layers F.Cu F.Paste F.Mask))
  (pad L2 smd circle (at -8.5 0.5) (size 0.5 0.5) (layers F.Cu F.Paste F.Mask))
  (pad L3 smd circle (at -7.5 0.5) (size 0.5 0.5) (layers F.Cu F.Paste F.Mask))
  (pad L4 smd circle (at -6.5 0.5) (size 0.5 0.5) (layers F.Cu F.Paste F.Mask))
  (pad K4 smd circle (at -6.5 -0.5) (size 0.5 0.5) (layers F.Cu F.Paste F.Mask))
  (pad K3 smd circle (at -7.5 -0.5) (size 0.5 0.5) (layers F.Cu F.Paste F.Mask))
  (pad K2 smd circle (at -8.5 -0.5) (size 0.5 0.5) (layers F.Cu F.Paste F.Mask))
  (pad K1 smd circle (at -9.5 -0.5) (size 0.5 0.5) (layers F.Cu F.Paste F.Mask))
  (pad J2 smd circle (at -8.5 -1.5) (size 0.5 0.5) (layers F.Cu F.Paste F.Mask))
  (pad J3 smd circle (at -7.5 -1.5) (size 0.5 0.5) (layers F.Cu F.Paste F.Mask))
  (pad J4 smd circle (at -6.5 -1.5) (size 0.5 0.5) (layers F.Cu F.Paste F.Mask))
  (pad H4 smd circle (at -6.5 -2.5) (size 0.5 0.5) (layers F.Cu F.Paste F.Mask))
  (pad H3 smd circle (at -7.5 -2.5) (size 0.5 0.5) (layers F.Cu F.Paste F.Mask))
  (pad H2 smd circle (at -8.5 -2.5) (size 0.5 0.5) (layers F.Cu F.Paste F.Mask))
  (pad G2 smd circle (at -8.5 -3.5) (size 0.5 0.5) (layers F.Cu F.Paste F.Mask))
  (pad G3 smd circle (at -7.5 -3.5) (size 0.5 0.5) (layers F.Cu F.Paste F.Mask))
  (pad G4 smd circle (at -6.5 -3.5) (size 0.5 0.5) (layers F.Cu F.Paste F.Mask))
  (pad F4 smd circle (at -6.5 -4.5) (size 0.5 0.5) (layers F.Cu F.Paste F.Mask))
  (pad F3 smd circle (at -7.5 -4.5) (size 0.5 0.5) (layers F.Cu F.Paste F.Mask))
  (pad F2 smd circle (at -8.5 -4.5) (size 0.5 0.5) (layers F.Cu F.Paste F.Mask))
  (pad E16 smd circle (at 5.5 -5.5) (size 0.5 0.5) (layers F.Cu F.Paste F.Mask))
  (pad F16 smd circle (at 5.5 -4.5) (size 0.5 0.5) (layers F.Cu F.Paste F.Mask))
  (pad G16 smd circle (at 5.5 -3.5) (size 0.5 0.5) (layers F.Cu F.Paste F.Mask))
  (pad G15 smd circle (at 4.5 -3.5) (size 0.5 0.5) (layers F.Cu F.Paste F.Mask))
  (pad F15 smd circle (at 4.5 -4.5) (size 0.5 0.5) (layers F.Cu F.Paste F.Mask))
  (pad E15 smd circle (at 4.5 -5.5) (size 0.5 0.5) (layers F.Cu F.Paste F.Mask))
  (pad E14 smd circle (at 3.5 -5.5) (size 0.5 0.5) (layers F.Cu F.Paste F.Mask))
  (pad F14 smd circle (at 3.5 -4.5) (size 0.5 0.5) (layers F.Cu F.Paste F.Mask))
  (pad F13 smd circle (at 2.5 -4.5) (size 0.5 0.5) (layers F.Cu F.Paste F.Mask))
  (pad E13 smd circle (at 2.5 -5.5) (size 0.5 0.5) (layers F.Cu F.Paste F.Mask))
  (pad C16 smd circle (at 5.5 -7.5) (size 0.5 0.5) (layers F.Cu F.Paste F.Mask))
  (pad D16 smd circle (at 5.5 -6.5) (size 0.5 0.5) (layers F.Cu F.Paste F.Mask))
  (pad D15 smd circle (at 4.5 -6.5) (size 0.5 0.5) (layers F.Cu F.Paste F.Mask))
  (pad C15 smd circle (at 4.5 -7.5) (size 0.5 0.5) (layers F.Cu F.Paste F.Mask))
  (pad D13 smd circle (at 2.5 -6.5) (size 0.5 0.5) (layers F.Cu F.Paste F.Mask))
  (pad D14 smd circle (at 3.5 -6.5) (size 0.5 0.5) (layers F.Cu F.Paste F.Mask))
  (pad C14 smd circle (at 3.5 -7.5) (size 0.5 0.5) (layers F.Cu F.Paste F.Mask))
  (pad C13 smd circle (at 2.5 -7.5) (size 0.5 0.5) (layers F.Cu F.Paste F.Mask))
  (pad C12 smd circle (at 1.5 -7.5) (size 0.5 0.5) (layers F.Cu F.Paste F.Mask))
  (pad D12 smd circle (at 1.5 -6.5) (size 0.5 0.5) (layers F.Cu F.Paste F.Mask))
  (pad D11 smd circle (at 0.5 -6.5) (size 0.5 0.5) (layers F.Cu F.Paste F.Mask))
  (pad C11 smd circle (at 0.5 -7.5) (size 0.5 0.5) (layers F.Cu F.Paste F.Mask))
  (pad D10 smd circle (at -0.5 -6.5) (size 0.5 0.5) (layers F.Cu F.Paste F.Mask))
  (pad C10 smd circle (at -0.5 -7.5) (size 0.5 0.5) (layers F.Cu F.Paste F.Mask))
  (pad E4 smd circle (at -6.5 -5.5) (size 0.5 0.5) (layers F.Cu F.Paste F.Mask))
  (pad E3 smd circle (at -7.5 -5.5) (size 0.5 0.5) (layers F.Cu F.Paste F.Mask))
  (pad E2 smd circle (at -8.5 -5.5) (size 0.5 0.5) (layers F.Cu F.Paste F.Mask))
  (pad D9 smd circle (at -1.5 -6.5) (size 0.5 0.5) (layers F.Cu F.Paste F.Mask))
  (pad D8 smd circle (at -2.5 -6.5) (size 0.5 0.5) (layers F.Cu F.Paste F.Mask))
  (pad D7 smd circle (at -3.5 -6.5) (size 0.5 0.5) (layers F.Cu F.Paste F.Mask))
  (pad D6 smd circle (at -4.5 -6.5) (size 0.5 0.5) (layers F.Cu F.Paste F.Mask))
  (pad D5 smd circle (at -5.5 -6.5) (size 0.5 0.5) (layers F.Cu F.Paste F.Mask))
  (pad D4 smd circle (at -6.5 -6.5) (size 0.5 0.5) (layers F.Cu F.Paste F.Mask))
  (pad D3 smd circle (at -7.5 -6.5) (size 0.5 0.5) (layers F.Cu F.Paste F.Mask))
  (pad D2 smd circle (at -8.5 -6.5) (size 0.5 0.5) (layers F.Cu F.Paste F.Mask))
  (pad C9 smd circle (at -1.5 -7.5) (size 0.5 0.5) (layers F.Cu F.Paste F.Mask))
  (pad C8 smd circle (at -2.5 -7.5) (size 0.5 0.5) (layers F.Cu F.Paste F.Mask))
  (pad C7 smd circle (at -3.5 -7.5) (size 0.5 0.5) (layers F.Cu F.Paste F.Mask))
  (pad C6 smd circle (at -4.5 -7.5) (size 0.5 0.5) (layers F.Cu F.Paste F.Mask))
  (pad C5 smd circle (at -5.5 -7.5) (size 0.5 0.5) (layers F.Cu F.Paste F.Mask))
  (pad C4 smd circle (at -6.5 -7.5) (size 0.5 0.5) (layers F.Cu F.Paste F.Mask))
  (pad C3 smd circle (at -7.5 -7.5) (size 0.5 0.5) (layers F.Cu F.Paste F.Mask))
  (pad C2 smd circle (at -8.5 -7.5) (size 0.5 0.5) (layers F.Cu F.Paste F.Mask))
  (pad B4 smd circle (at -6.5 -8.5) (size 0.5 0.5) (layers F.Cu F.Paste F.Mask))
  (pad B3 smd circle (at -7.5 -8.5) (size 0.5 0.5) (layers F.Cu F.Paste F.Mask))
  (pad B2 smd circle (at -8.5 -8.5) (size 0.5 0.5) (layers F.Cu F.Paste F.Mask))
  (pad B5 smd circle (at -5.5 -8.5) (size 0.5 0.5) (layers F.Cu F.Paste F.Mask))
  (pad B6 smd circle (at -4.5 -8.5) (size 0.5 0.5) (layers F.Cu F.Paste F.Mask))
  (pad B7 smd circle (at -3.5 -8.5) (size 0.5 0.5) (layers F.Cu F.Paste F.Mask))
  (pad B8 smd circle (at -2.5 -8.5) (size 0.5 0.5) (layers F.Cu F.Paste F.Mask))
  (pad B9 smd circle (at -1.5 -8.5) (size 0.5 0.5) (layers F.Cu F.Paste F.Mask))
  (pad B10 smd circle (at -0.5 -8.5) (size 0.5 0.5) (layers F.Cu F.Paste F.Mask))
  (pad B11 smd circle (at 0.5 -8.5) (size 0.5 0.5) (layers F.Cu F.Paste F.Mask))
  (pad B12 smd circle (at 1.5 -8.5) (size 0.5 0.5) (layers F.Cu F.Paste F.Mask))
  (pad B13 smd circle (at 2.5 -8.5) (size 0.5 0.5) (layers F.Cu F.Paste F.Mask))
  (pad B14 smd circle (at 3.5 -8.5) (size 0.5 0.5) (layers F.Cu F.Paste F.Mask))
  (pad B15 smd circle (at 4.5 -8.5) (size 0.5 0.5) (layers F.Cu F.Paste F.Mask))
  (pad B16 smd circle (at 5.5 -8.5) (size 0.5 0.5) (layers F.Cu F.Paste F.Mask))
  (pad J1 smd circle (at -9.5 -1.5) (size 0.5 0.5) (layers F.Cu F.Paste F.Mask))
  (pad H1 smd circle (at -9.5 -2.5) (size 0.5 0.5) (layers F.Cu F.Paste F.Mask))
  (pad G1 smd circle (at -9.5 -3.5) (size 0.5 0.5) (layers F.Cu F.Paste F.Mask))
  (pad F1 smd circle (at -9.5 -4.5) (size 0.5 0.5) (layers F.Cu F.Paste F.Mask))
  (pad E1 smd circle (at -9.5 -5.5) (size 0.5 0.5) (layers F.Cu F.Paste F.Mask))
  (pad D1 smd circle (at -9.5 -6.5) (size 0.5 0.5) (layers F.Cu F.Paste F.Mask))
  (pad C1 smd circle (at -9.5 -7.5) (size 0.5 0.5) (layers F.Cu F.Paste F.Mask))
  (pad B1 smd circle (at -9.5 -8.5) (size 0.5 0.5) (layers F.Cu F.Paste F.Mask))
  (pad A16 smd circle (at 5.5 -9.5) (size 0.5 0.5) (layers F.Cu F.Paste F.Mask))
  (pad A15 smd circle (at 4.5 -9.5) (size 0.5 0.5) (layers F.Cu F.Paste F.Mask))
  (pad A14 smd circle (at 3.5 -9.5) (size 0.5 0.5) (layers F.Cu F.Paste F.Mask))
  (pad A13 smd circle (at 2.5 -9.5) (size 0.5 0.5) (layers F.Cu F.Paste F.Mask))
  (pad A12 smd circle (at 1.5 -9.5) (size 0.5 0.5) (layers F.Cu F.Paste F.Mask))
  (pad A11 smd circle (at 0.5 -9.5) (size 0.5 0.5) (layers F.Cu F.Paste F.Mask))
  (pad A10 smd circle (at -0.5 -9.5) (size 0.5 0.5) (layers F.Cu F.Paste F.Mask))
  (pad A9 smd circle (at -1.5 -9.5) (size 0.5 0.5) (layers F.Cu F.Paste F.Mask))
  (pad A8 smd circle (at -2.5 -9.5) (size 0.5 0.5) (layers F.Cu F.Paste F.Mask))
  (pad A7 smd circle (at -3.5 -9.5) (size 0.5 0.5) (layers F.Cu F.Paste F.Mask))
  (pad A6 smd circle (at -4.5 -9.5) (size 0.5 0.5) (layers F.Cu F.Paste F.Mask))
  (pad A5 smd circle (at -5.5 -9.5) (size 0.5 0.5) (layers F.Cu F.Paste F.Mask))
  (pad A4 smd circle (at -6.5 -9.5) (size 0.5 0.5) (layers F.Cu F.Paste F.Mask))
  (pad A3 smd circle (at -7.5 -9.5) (size 0.5 0.5) (layers F.Cu F.Paste F.Mask))
  (pad A2 smd circle (at -8.5 -9.5) (size 0.5 0.5) (layers F.Cu F.Paste F.Mask))
  (pad A1 smd circle (at -9.5 -9.5) (size 0.5 0.5) (layers F.Cu F.Paste F.Mask)))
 (gr_line (start 90 40) (end 90 15) (layer Edge.Cuts) (width 0.05))
 (gr_line (start 130 40) (end 90 40) (layer Edge.Cuts) (width 0.05))
 (gr_line (start 130 15) (end 130 40) (layer Edge.Cuts) (width 0.05))
 (gr_line (start 90 15) (end 130 15) (layer Edge.Cuts) (width 0.05))
 (segment (start 117.4 21.5) (end 113.7 25.2) (width 0.25) (layer F.Cu) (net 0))
 (segment (start 117.5 21.5) (end 117.4 21.5) (width 0.25) (layer F.Cu) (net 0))
 (segment (start 117.5 29.5) (end 117.5 26.5) (width 0.25) (layer F.Cu) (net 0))
 (segment (start 117.5 26.5) (end 121.6 22.4) (width 0.25) (layer F.Cu) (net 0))
 (segment (start 121.6 22.4) (end 121.6 19.1) (width 0.25) (layer F.Cu) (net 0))
 (segment (start 121.6 19.1) (end 120.2 17.7) (width 0.25) (layer F.Cu) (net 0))
 (segment (start 120.2 17.7) (end 112 17.7) (width 0.25) (layer F.Cu) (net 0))
 (segment (start 109.5 20.2) (end 109.5 21.5) (width 0.25) (layer F.Cu) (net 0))
 (segment (start 112 17.7) (end 109.5 20.2) (width 0.25) (layer F.Cu) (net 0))
 (segment (start 113.7 25.3) (end 109.5 29.5) (width 0.25) (layer B.Cu) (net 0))
 (segment (start 113.7 25.2) (end 113.7 25.3) (width 0.25) (layer B.Cu) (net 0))
 (segment (start 97.2 33.7) (end 97.2 33.7) (width 0.25) (layer F.Cu) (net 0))
 (segment (start 111.6 33.7) (end 120.5 33.7) (width 0.25) (layer F.Cu) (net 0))
 (segment (start 120.5 33.7) (end 120.5 28.8) (width 0.25) (layer F.Cu) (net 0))
 (segment (start 120.5 28.8) (end 122.9 31.2) (width 0.25) (layer F.Cu) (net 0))
 (segment (start 122.9 31.2) (end 122.9 31.6) (width 0.25) (layer F.Cu) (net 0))
 (segment (start 122.9 31.6) (end 126.5 35.2) (width 0.25) (layer F.Cu) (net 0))
 (segment (start 126.5 35.2) (end 126.9 35.2) (width 0.25) (layer F.Cu) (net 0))
 (segment (start 126.9 35.2) (end 126.9 35.2) (width 0.25) (layer F.Cu) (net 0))
 (via (at 126.9 35.2) (size 0.8) (drill 0.4) (layers F.Cu B.Cu) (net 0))
 (segment (start 97.2 33.7) (end 111.6 33.7) (width 0.25) (layer F.Cu) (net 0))
 (via (at 97.2 33.7) (size 0.8) (drill 0.4) (layers F.Cu B.Cu) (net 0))
 (segment (start 101.4 29.5) (end 97.2 33.7) (width 0.25) (layer F.Cu) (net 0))
 (segment (start 109.5 29.5) (end 101.4 29.5) (width 0.25) (layer F.Cu) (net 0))
 (segment (start 126.9 35.2) (end 95.7 35.2) (width 0.25) (layer F.Cu) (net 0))
 (segment (start 93.85 33.35) (end 93.85 27.15) (width 0.25) (layer F.Cu) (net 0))
 (segment (start 95.7 35.2) (end 93.85 33.35) (width 0.25) (layer F.Cu) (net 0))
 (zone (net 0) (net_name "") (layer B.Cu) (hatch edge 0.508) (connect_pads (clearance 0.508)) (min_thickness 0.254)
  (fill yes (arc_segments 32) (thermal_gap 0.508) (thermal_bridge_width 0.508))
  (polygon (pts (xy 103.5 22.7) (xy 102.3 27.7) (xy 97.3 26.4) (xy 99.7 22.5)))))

